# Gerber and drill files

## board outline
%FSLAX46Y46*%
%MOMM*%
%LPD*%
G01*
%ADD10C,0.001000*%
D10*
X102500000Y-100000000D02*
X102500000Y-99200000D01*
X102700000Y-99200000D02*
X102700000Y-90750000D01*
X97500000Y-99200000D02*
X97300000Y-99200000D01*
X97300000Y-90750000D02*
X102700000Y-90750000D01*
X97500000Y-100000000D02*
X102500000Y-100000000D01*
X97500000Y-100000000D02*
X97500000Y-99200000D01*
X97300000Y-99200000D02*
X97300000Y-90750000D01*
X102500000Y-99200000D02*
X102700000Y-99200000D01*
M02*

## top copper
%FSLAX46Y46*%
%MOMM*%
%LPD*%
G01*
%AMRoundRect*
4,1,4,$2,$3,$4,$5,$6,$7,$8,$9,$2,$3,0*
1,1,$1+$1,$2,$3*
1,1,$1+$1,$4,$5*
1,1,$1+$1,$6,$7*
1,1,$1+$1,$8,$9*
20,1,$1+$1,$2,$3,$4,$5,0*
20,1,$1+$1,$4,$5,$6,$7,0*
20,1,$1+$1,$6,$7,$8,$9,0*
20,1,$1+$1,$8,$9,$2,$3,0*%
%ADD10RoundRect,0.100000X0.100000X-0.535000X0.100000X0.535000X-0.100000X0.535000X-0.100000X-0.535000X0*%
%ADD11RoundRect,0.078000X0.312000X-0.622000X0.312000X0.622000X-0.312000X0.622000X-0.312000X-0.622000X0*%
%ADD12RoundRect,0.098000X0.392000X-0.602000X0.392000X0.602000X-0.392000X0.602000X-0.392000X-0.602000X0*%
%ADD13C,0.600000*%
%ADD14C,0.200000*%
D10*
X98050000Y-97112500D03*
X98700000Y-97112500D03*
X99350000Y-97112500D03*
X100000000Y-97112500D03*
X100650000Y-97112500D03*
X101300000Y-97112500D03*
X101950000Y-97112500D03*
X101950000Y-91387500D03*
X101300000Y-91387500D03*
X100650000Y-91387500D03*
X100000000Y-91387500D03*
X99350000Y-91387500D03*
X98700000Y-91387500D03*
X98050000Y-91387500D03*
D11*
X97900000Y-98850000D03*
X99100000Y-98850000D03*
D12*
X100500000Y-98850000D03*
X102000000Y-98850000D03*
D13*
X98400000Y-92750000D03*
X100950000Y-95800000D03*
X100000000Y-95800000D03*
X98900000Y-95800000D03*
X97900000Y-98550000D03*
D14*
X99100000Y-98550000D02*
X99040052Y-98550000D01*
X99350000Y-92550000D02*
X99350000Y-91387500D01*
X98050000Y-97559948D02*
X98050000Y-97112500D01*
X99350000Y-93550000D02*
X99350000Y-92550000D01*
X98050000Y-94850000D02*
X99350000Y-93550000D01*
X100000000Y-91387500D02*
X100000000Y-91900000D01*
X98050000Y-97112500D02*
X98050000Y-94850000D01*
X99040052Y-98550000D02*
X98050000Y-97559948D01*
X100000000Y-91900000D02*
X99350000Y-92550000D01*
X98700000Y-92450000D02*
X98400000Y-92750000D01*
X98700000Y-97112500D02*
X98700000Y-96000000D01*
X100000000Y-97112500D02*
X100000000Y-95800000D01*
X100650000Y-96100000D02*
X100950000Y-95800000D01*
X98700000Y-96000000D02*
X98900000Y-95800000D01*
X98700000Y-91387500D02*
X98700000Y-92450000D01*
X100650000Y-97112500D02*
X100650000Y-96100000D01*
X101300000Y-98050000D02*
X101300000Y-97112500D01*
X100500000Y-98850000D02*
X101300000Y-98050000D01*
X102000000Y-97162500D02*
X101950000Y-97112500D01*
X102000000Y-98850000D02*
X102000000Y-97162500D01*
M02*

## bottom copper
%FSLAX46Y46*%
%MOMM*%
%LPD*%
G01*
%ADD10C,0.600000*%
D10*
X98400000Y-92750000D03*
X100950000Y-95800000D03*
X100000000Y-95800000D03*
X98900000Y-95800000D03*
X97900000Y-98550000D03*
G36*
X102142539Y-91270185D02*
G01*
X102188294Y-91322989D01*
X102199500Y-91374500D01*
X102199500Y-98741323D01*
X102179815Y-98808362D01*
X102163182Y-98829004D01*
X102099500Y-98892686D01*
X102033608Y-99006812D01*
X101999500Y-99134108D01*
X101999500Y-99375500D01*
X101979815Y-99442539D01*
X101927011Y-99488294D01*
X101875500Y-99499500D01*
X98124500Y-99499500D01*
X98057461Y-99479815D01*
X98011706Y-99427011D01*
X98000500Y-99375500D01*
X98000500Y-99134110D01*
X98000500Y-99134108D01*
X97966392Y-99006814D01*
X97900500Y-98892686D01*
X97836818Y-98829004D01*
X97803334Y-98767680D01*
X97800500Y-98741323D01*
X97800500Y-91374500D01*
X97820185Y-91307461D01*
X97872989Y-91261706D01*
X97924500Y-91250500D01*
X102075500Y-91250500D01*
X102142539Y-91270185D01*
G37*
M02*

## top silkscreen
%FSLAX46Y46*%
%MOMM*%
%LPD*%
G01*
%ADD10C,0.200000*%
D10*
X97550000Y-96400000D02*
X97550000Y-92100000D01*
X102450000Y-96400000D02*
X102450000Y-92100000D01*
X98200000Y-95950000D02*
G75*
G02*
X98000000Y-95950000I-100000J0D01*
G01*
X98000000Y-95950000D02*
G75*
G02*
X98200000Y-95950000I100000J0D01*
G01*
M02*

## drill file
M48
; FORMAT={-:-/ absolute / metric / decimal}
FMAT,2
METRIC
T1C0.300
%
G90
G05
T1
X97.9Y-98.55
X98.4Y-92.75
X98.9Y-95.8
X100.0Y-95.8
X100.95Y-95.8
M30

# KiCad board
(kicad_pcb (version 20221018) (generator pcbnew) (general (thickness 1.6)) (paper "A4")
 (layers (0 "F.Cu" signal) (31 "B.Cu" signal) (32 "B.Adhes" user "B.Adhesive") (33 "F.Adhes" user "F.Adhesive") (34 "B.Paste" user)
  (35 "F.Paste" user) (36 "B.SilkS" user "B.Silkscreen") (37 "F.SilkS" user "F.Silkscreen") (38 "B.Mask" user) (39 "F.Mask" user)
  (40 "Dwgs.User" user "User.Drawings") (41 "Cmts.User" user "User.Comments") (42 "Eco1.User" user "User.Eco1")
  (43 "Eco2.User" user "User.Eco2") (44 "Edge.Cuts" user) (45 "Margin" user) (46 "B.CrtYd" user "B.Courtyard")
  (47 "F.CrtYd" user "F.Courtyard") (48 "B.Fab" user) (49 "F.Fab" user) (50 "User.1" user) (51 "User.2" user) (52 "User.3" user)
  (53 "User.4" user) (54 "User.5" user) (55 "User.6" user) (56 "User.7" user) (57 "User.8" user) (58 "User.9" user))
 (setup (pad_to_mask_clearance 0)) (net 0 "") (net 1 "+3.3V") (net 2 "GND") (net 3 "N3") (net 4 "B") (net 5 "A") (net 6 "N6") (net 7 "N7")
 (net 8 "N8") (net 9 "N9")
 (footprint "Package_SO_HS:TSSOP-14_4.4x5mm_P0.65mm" (layer "F.Cu") (at 100 94.25 90)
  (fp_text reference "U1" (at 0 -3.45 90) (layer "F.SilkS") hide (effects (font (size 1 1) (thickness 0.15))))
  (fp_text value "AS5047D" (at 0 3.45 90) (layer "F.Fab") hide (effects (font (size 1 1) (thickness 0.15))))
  (fp_line (start -2.15 -2.45) (end 2.15 -2.45) (stroke (width 0.2) (type default)) (layer "F.SilkS"))
  (fp_line (start -2.15 2.45) (end 2.15 2.45) (stroke (width 0.2) (type default)) (layer "F.SilkS"))
  (fp_circle (center -1.7 -1.9) (end -1.7 -1.8) (stroke (width 0.2) (type default)) (fill none) (layer "F.SilkS"))
  (pad "1" smd roundrect (at -2.8625 -1.95 90) (size 1.27 0.4) (layers "F.Cu" "F.Paste" "F.Mask") (roundrect_rratio 0.25) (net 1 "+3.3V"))
  (pad "2" smd roundrect (at -2.8625 -1.3 90) (size 1.27 0.4) (layers "F.Cu" "F.Paste" "F.Mask") (roundrect_rratio 0.25) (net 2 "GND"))
  (pad "3" smd roundrect (at -2.8625 -0.65 90) (size 1.27 0.4) (layers "F.Cu" "F.Paste" "F.Mask") (roundrect_rratio 0.25) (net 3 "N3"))
  (pad "4" smd roundrect (at -2.8625 0 90) (size 1.27 0.4) (layers "F.Cu" "F.Paste" "F.Mask") (roundrect_rratio 0.25) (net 2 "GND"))
  (pad "5" smd roundrect (at -2.8625 0.65 90) (size 1.27 0.4) (layers "F.Cu" "F.Paste" "F.Mask") (roundrect_rratio 0.25) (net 2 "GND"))
  (pad "6" smd roundrect (at -2.8625 1.3 90) (size 1.27 0.4) (layers "F.Cu" "F.Paste" "F.Mask") (roundrect_rratio 0.25) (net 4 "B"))
  (pad "7" smd roundrect (at -2.8625 1.95 90) (size 1.27 0.4) (layers "F.Cu" "F.Paste" "F.Mask") (roundrect_rratio 0.25) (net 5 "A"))
  (pad "8" smd roundrect (at 2.8625 1.95 90) (size 1.27 0.4) (layers "F.Cu" "F.Paste" "F.Mask") (roundrect_rratio 0.25) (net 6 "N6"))
  (pad "9" smd roundrect (at 2.8625 1.3 90) (size 1.27 0.4) (layers "F.Cu" "F.Paste" "F.Mask") (roundrect_rratio 0.25) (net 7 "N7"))
  (pad "10" smd roundrect (at 2.8625 0.65 90) (size 1.27 0.4) (layers "F.Cu" "F.Paste" "F.Mask") (roundrect_rratio 0.25) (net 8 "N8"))
  (pad "11" smd roundrect (at 2.8625 0 90) (size 1.27 0.4) (layers "F.Cu" "F.Paste" "F.Mask") (roundrect_rratio 0.25) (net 1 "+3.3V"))
  (pad "12" smd roundrect (at 2.8625 -0.65 90) (size 1.27 0.4) (layers "F.Cu" "F.Paste" "F.Mask") (roundrect_rratio 0.25) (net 1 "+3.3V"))
  (pad "13" smd roundrect (at 2.8625 -1.3 90) (size 1.27 0.4) (layers "F.Cu" "F.Paste" "F.Mask") (roundrect_rratio 0.25) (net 2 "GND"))
  (pad "14" smd roundrect (at 2.8625 -1.95 90) (size 1.27 0.4) (layers "F.Cu" "F.Paste" "F.Mask") (roundrect_rratio 0.25) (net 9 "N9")))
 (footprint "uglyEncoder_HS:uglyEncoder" (layer "F.Cu") (at 100 99.55)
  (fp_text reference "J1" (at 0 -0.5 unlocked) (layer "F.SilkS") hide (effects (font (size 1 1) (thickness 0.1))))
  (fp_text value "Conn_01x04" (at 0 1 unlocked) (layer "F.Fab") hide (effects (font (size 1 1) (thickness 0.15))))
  (pad "1" smd roundrect (at -2.1 -0.7 90) (size 1.4 0.78) (layers "F.Cu" "F.Paste" "F.Mask") (roundrect_rratio 0.1) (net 2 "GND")
   (thermal_bridge_angle 45))
  (pad "2" smd roundrect (at -0.9 -0.7 90) (size 1.4 0.78) (layers "F.Cu" "F.Paste" "F.Mask") (roundrect_rratio 0.1) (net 1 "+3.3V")
   (thermal_bridge_angle 45))
  (pad "3" smd roundrect (at 0.5 -0.7 90) (size 1.4 0.98) (layers "F.Cu" "F.Paste" "F.Mask") (roundrect_rratio 0.1) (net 4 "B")
   (thermal_bridge_angle 45))
  (pad "4" smd roundrect (at 2 -0.7 90) (size 1.4 0.98) (layers "F.Cu" "F.Paste" "F.Mask") (roundrect_rratio 0.1) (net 5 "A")
   (thermal_bridge_angle 45)))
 (gr_line (start 102.5 100) (end 102.5 99.2) (stroke (width 0.001) (type solid)) (layer "Edge.Cuts"))
 (gr_line (start 102.7 99.2) (end 102.7 90.75) (stroke (width 0.001) (type solid)) (layer "Edge.Cuts"))
 (gr_line (start 97.5 99.2) (end 97.3 99.2) (stroke (width 0.001) (type solid)) (layer "Edge.Cuts"))
 (gr_line (start 97.3 90.75) (end 102.7 90.75) (stroke (width 0.001) (type solid)) (layer "Edge.Cuts"))
 (gr_line (start 97.5 100) (end 102.5 100) (stroke (width 0.001) (type solid)) (layer "Edge.Cuts"))
 (gr_line (start 97.5 100) (end 97.5 99.2) (stroke (width 0.001) (type solid)) (layer "Edge.Cuts"))
 (gr_line (start 97.3 99.2) (end 97.3 90.75) (stroke (width 0.001) (type solid)) (layer "Edge.Cuts"))
 (gr_line (start 102.5 99.2) (end 102.7 99.2) (stroke (width 0.001) (type solid)) (layer "Edge.Cuts"))
 (segment (start 99.1 98.55) (end 99.040052 98.55) (width 0.2) (layer "F.Cu") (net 1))
 (segment (start 99.35 92.55) (end 99.35 91.3875) (width 0.2) (layer "F.Cu") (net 1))
 (segment (start 98.05 97.559948) (end 98.05 97.1125) (width 0.2) (layer "F.Cu") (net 1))
 (segment (start 99.35 93.55) (end 99.35 92.55) (width 0.2) (layer "F.Cu") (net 1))
 (segment (start 98.05 94.85) (end 99.35 93.55) (width 0.2) (layer "F.Cu") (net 1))
 (segment (start 100 91.3875) (end 100 91.9) (width 0.2) (layer "F.Cu") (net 1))
 (segment (start 98.05 97.1125) (end 98.05 94.85) (width 0.2) (layer "F.Cu") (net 1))
 (segment (start 99.040052 98.55) (end 98.05 97.559948) (width 0.2) (layer "F.Cu") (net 1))
 (segment (start 100 91.9) (end 99.35 92.55) (width 0.2) (layer "F.Cu") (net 1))
 (segment (start 98.7 92.45) (end 98.4 92.75) (width 0.2) (layer "F.Cu") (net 2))
 (segment (start 98.7 97.1125) (end 98.7 96) (width 0.2) (layer "F.Cu") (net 2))
 (segment (start 100 97.1125) (end 100 95.8) (width 0.2) (layer "F.Cu") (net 2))
 (segment (start 100.65 96.1) (end 100.95 95.8) (width 0.2) (layer "F.Cu") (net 2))
 (segment (start 98.7 96) (end 98.9 95.8) (width 0.2) (layer "F.Cu") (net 2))
 (segment (start 98.7 91.3875) (end 98.7 92.45) (width 0.2) (layer "F.Cu") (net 2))
 (segment (start 100.65 97.1125) (end 100.65 96.1) (width 0.2) (layer "F.Cu") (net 2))
 (via (at 98.4 92.75) (size 0.6) (drill 0.3) (layers "F.Cu" "B.Cu") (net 2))
 (via (at 100.95 95.8) (size 0.6) (drill 0.3) (layers "F.Cu" "B.Cu") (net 2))
 (via (at 100 95.8) (size 0.6) (drill 0.3) (layers "F.Cu" "B.Cu") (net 2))
 (via (at 98.9 95.8) (size 0.6) (drill 0.3) (layers "F.Cu" "B.Cu") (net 2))
 (via (at 97.9 98.55) (size 0.6) (drill 0.3) (layers "F.Cu" "B.Cu") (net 2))
 (segment (start 101.3 98.05) (end 101.3 97.1125) (width 0.2) (layer "F.Cu") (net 4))
 (segment (start 100.5 98.85) (end 101.3 98.05) (width 0.2) (layer "F.Cu") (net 4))
 (segment (start 102 97.1625) (end 101.95 97.1125) (width 0.2) (layer "F.Cu") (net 5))
 (segment (start 102 98.85) (end 102 97.1625) (width 0.2) (layer "F.Cu") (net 5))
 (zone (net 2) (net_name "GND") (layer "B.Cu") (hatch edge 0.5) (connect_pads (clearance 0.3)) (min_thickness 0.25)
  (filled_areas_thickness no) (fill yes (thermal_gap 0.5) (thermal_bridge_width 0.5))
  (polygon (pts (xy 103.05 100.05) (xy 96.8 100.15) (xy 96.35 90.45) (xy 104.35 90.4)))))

